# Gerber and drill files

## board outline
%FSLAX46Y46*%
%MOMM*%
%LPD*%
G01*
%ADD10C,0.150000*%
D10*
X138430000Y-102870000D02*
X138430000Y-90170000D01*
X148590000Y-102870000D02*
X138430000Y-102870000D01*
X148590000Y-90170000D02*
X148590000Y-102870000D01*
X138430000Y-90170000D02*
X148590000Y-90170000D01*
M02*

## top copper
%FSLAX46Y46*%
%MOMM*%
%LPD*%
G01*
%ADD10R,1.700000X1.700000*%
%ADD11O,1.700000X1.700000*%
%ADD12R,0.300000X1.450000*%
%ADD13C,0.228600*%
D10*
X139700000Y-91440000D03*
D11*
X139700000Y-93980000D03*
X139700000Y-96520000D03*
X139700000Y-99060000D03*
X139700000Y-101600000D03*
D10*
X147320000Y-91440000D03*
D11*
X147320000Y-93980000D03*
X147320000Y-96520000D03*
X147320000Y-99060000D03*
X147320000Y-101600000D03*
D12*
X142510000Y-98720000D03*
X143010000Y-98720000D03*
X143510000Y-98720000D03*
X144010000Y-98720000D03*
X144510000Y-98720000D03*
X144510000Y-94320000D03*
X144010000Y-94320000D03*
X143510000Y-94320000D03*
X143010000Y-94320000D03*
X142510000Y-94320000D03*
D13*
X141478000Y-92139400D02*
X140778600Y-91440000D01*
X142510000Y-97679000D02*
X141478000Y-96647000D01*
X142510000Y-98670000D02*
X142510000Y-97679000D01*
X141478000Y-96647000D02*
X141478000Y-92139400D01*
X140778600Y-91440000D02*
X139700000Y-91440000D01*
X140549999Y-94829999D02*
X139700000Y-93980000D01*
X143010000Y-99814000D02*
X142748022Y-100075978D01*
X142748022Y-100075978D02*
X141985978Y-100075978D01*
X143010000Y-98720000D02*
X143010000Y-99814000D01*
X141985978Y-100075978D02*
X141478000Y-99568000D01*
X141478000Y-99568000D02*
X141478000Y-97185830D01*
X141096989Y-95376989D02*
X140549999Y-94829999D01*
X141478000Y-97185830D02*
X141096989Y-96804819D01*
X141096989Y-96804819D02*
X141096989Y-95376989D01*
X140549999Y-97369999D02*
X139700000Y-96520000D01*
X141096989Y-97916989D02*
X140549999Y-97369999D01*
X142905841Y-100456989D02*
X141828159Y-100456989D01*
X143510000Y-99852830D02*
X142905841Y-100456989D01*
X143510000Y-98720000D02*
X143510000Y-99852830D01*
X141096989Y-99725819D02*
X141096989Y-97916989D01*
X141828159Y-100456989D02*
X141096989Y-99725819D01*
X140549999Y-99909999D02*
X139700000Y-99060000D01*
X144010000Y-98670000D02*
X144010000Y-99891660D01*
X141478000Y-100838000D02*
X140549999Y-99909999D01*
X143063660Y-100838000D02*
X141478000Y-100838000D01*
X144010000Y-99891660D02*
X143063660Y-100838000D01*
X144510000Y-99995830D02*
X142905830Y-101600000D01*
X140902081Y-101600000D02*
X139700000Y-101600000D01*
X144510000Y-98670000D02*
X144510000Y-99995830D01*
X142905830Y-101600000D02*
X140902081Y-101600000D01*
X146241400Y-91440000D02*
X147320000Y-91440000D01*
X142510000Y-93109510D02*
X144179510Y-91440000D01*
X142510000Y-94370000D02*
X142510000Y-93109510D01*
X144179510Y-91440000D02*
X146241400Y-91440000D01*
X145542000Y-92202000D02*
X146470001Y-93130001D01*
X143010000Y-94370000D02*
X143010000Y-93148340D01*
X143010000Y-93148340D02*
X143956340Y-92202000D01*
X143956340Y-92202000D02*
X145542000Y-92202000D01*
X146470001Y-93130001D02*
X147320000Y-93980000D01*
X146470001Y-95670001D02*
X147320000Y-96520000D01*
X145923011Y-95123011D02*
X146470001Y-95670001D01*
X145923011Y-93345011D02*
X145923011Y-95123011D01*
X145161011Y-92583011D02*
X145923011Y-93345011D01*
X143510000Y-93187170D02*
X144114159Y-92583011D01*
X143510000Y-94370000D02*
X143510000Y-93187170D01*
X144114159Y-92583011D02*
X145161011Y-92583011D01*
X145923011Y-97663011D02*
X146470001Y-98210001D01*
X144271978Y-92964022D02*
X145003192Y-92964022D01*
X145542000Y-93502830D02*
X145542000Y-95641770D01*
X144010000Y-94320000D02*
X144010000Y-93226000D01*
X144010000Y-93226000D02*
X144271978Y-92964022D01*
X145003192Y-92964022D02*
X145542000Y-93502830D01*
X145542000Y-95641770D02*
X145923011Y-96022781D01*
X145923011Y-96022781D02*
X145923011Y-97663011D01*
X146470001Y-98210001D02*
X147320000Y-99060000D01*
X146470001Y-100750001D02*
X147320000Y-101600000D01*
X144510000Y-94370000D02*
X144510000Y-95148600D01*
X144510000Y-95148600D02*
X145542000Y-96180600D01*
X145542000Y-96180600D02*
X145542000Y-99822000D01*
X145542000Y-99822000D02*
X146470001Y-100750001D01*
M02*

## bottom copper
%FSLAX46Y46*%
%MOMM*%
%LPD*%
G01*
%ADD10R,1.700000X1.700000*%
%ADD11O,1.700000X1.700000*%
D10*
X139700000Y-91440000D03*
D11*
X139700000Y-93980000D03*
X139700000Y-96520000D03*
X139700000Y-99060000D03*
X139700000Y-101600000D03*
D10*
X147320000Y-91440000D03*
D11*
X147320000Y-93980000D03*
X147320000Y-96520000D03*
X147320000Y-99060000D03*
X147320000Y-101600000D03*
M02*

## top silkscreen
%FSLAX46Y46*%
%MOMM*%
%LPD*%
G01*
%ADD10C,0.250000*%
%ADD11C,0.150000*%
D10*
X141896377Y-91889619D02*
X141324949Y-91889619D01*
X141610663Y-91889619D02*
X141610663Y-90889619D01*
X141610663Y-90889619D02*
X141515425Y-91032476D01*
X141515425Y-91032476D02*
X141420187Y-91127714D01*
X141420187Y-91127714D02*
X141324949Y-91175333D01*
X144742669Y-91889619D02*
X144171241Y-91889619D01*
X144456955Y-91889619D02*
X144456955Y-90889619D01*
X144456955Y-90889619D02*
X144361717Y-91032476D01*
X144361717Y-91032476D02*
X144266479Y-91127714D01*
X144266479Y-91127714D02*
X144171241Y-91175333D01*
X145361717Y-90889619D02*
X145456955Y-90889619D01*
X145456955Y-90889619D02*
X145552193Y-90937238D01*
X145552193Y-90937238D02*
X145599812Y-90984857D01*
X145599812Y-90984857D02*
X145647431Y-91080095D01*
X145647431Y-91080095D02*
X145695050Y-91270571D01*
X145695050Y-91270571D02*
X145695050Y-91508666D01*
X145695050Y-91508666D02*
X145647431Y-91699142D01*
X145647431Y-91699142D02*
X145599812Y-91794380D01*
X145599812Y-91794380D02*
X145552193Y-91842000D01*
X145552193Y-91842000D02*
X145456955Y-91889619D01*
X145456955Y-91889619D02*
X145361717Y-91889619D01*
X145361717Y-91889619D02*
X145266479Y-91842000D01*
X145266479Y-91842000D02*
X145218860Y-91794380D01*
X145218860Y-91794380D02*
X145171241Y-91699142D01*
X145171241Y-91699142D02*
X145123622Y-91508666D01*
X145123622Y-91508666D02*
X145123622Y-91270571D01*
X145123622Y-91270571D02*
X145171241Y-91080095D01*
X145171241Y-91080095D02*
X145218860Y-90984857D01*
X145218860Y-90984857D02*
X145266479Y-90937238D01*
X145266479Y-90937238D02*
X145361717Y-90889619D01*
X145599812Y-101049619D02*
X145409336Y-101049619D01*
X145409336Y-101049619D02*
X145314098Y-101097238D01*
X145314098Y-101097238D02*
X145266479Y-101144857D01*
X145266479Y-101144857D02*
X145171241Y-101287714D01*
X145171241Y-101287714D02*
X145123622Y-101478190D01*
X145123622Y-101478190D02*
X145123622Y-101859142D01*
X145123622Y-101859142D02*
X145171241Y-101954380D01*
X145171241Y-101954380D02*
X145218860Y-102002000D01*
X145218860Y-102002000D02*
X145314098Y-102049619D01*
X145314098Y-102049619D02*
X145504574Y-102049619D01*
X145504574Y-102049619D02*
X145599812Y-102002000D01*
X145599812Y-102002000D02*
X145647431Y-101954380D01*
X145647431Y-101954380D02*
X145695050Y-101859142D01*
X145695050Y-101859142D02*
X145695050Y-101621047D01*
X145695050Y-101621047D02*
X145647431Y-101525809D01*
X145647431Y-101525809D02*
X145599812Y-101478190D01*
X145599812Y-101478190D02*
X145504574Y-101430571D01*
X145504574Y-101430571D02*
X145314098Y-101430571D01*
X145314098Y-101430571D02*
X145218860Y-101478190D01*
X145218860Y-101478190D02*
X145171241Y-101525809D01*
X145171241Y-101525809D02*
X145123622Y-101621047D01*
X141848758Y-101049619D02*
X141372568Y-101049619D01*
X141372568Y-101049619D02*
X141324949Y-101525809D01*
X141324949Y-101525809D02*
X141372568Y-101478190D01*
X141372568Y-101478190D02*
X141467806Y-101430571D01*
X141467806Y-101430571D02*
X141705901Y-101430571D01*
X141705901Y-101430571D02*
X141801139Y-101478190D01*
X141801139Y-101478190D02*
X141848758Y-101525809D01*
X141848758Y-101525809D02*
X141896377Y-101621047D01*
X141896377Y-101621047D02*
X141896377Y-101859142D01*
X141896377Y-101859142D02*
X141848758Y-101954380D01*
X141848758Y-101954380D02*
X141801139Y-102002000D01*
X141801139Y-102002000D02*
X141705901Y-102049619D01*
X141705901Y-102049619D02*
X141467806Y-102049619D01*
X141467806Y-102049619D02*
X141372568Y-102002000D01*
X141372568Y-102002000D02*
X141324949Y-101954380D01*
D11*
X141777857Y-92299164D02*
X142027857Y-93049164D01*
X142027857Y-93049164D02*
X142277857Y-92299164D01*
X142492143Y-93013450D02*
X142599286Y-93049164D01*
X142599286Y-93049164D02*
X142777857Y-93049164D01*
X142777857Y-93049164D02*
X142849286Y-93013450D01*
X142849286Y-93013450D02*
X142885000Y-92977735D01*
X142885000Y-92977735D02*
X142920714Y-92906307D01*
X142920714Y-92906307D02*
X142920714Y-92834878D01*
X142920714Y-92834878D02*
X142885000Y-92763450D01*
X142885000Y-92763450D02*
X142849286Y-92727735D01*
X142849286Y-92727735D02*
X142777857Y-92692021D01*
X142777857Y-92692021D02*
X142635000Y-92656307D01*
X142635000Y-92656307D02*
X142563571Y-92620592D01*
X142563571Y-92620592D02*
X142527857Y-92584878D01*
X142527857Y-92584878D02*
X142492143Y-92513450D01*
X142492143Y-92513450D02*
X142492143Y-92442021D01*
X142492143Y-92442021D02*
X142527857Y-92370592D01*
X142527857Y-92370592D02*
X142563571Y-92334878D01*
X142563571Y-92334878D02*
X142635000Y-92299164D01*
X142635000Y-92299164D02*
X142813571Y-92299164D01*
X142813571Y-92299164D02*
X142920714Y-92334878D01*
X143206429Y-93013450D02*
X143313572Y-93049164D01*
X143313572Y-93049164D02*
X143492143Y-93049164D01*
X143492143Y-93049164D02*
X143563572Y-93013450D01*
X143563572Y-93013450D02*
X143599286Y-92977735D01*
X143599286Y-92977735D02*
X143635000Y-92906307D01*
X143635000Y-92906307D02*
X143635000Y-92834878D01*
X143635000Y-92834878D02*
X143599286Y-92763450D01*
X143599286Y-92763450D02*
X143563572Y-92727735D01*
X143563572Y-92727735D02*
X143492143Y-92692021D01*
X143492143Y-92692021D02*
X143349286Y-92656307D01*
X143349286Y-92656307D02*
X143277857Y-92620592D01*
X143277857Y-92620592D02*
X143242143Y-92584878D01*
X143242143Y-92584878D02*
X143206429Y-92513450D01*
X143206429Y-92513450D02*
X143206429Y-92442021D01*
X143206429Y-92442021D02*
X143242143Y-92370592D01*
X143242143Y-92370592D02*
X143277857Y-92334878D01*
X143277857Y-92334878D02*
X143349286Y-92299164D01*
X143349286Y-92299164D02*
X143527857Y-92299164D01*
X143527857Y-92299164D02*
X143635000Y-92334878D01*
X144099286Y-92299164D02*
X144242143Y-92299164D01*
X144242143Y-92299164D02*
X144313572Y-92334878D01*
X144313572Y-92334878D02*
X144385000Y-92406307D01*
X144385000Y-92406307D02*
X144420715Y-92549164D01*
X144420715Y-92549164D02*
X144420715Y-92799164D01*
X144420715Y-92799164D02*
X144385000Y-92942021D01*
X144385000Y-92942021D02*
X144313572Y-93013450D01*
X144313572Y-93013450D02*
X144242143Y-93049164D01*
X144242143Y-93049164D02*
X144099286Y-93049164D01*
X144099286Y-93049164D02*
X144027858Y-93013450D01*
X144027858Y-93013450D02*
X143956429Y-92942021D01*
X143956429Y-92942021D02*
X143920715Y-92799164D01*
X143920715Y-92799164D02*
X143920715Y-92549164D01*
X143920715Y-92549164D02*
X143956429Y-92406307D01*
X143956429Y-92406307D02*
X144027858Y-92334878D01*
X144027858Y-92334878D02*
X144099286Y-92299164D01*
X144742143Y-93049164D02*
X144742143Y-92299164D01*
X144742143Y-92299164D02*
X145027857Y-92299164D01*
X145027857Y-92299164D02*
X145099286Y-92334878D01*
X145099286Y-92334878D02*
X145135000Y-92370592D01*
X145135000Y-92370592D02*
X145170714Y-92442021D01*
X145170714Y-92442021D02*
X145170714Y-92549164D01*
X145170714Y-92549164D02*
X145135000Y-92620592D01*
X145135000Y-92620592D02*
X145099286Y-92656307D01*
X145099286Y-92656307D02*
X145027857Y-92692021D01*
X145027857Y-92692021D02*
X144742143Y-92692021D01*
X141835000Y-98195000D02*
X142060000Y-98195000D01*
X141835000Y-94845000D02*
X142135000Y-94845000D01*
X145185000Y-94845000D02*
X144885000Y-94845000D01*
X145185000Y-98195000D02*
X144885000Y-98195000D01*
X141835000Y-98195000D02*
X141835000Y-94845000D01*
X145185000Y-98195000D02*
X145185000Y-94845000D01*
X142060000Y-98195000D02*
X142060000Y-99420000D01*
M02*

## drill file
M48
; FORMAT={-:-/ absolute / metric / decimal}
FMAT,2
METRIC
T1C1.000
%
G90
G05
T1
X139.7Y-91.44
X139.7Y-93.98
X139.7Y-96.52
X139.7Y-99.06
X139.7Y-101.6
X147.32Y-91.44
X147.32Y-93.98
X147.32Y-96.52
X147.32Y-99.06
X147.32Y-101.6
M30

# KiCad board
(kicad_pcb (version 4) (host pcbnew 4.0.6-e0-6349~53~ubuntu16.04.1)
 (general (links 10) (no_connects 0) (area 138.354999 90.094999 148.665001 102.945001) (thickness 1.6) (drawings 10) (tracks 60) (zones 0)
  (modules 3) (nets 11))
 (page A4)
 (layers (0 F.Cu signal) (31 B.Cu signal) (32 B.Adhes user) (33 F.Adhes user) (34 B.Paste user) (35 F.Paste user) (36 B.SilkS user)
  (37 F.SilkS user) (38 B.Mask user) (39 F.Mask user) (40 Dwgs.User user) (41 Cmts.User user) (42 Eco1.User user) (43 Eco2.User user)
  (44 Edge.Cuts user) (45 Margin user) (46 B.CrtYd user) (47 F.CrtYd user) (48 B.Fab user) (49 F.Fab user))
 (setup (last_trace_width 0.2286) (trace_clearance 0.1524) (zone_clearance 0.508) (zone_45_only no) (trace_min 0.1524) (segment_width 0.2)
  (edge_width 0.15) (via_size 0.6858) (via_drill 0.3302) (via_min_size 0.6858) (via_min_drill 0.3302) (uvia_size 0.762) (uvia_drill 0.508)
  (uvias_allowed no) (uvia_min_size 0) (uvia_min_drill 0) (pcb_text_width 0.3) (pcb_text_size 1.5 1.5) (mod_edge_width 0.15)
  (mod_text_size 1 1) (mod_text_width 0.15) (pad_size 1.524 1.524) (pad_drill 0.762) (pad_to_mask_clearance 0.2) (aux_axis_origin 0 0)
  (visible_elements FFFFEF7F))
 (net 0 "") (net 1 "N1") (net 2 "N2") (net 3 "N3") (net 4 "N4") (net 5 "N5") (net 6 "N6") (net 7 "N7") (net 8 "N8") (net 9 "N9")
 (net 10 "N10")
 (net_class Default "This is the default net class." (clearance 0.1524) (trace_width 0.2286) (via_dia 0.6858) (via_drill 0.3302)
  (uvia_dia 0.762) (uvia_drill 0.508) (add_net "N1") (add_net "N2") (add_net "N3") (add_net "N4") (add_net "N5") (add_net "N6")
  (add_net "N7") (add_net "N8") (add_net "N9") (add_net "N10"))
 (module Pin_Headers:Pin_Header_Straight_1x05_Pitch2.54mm (layer B.Cu) (at 139.7 91.44 180)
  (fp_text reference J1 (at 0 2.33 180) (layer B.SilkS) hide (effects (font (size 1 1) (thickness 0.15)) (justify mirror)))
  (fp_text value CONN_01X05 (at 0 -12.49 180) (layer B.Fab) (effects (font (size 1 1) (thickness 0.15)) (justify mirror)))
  (pad 1 thru_hole rect (at 0 0 180) (size 1.7 1.7) (drill 1) (layers *.Cu *.Mask) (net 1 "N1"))
  (pad 2 thru_hole oval (at 0 -2.54 180) (size 1.7 1.7) (drill 1) (layers *.Cu *.Mask) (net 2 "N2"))
  (pad 3 thru_hole oval (at 0 -5.08 180) (size 1.7 1.7) (drill 1) (layers *.Cu *.Mask) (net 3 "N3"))
  (pad 4 thru_hole oval (at 0 -7.62 180) (size 1.7 1.7) (drill 1) (layers *.Cu *.Mask) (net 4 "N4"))
  (pad 5 thru_hole oval (at 0 -10.16 180) (size 1.7 1.7) (drill 1) (layers *.Cu *.Mask) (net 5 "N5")))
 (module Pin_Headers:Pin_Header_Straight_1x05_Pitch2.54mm (layer B.Cu) (at 147.32 91.44 180)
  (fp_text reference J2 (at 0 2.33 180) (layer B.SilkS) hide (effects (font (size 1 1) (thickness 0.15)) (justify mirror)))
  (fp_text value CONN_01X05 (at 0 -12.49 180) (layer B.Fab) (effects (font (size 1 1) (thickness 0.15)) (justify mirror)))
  (pad 1 thru_hole rect (at 0 0 180) (size 1.7 1.7) (drill 1) (layers *.Cu *.Mask) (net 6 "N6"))
  (pad 2 thru_hole oval (at 0 -2.54 180) (size 1.7 1.7) (drill 1) (layers *.Cu *.Mask) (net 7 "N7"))
  (pad 3 thru_hole oval (at 0 -5.08 180) (size 1.7 1.7) (drill 1) (layers *.Cu *.Mask) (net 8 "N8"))
  (pad 4 thru_hole oval (at 0 -7.62 180) (size 1.7 1.7) (drill 1) (layers *.Cu *.Mask) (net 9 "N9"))
  (pad 5 thru_hole oval (at 0 -10.16 180) (size 1.7 1.7) (drill 1) (layers *.Cu *.Mask) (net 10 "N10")))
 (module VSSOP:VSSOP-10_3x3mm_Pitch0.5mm (layer F.Cu) (at 143.51 96.52 90)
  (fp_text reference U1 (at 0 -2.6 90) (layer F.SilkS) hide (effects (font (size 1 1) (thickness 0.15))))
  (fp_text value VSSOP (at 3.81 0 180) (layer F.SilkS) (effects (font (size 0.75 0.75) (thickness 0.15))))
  (fp_line (start -1.675 -1.675) (end -1.675 -1.45) (layer F.SilkS) (width 0.15))
  (fp_line (start 1.675 -1.675) (end 1.675 -1.375) (layer F.SilkS) (width 0.15))
  (fp_line (start 1.675 1.675) (end 1.675 1.375) (layer F.SilkS) (width 0.15))
  (fp_line (start -1.675 1.675) (end -1.675 1.375) (layer F.SilkS) (width 0.15))
  (fp_line (start -1.675 -1.675) (end 1.675 -1.675) (layer F.SilkS) (width 0.15))
  (fp_line (start -1.675 1.675) (end 1.675 1.675) (layer F.SilkS) (width 0.15))
  (fp_line (start -1.675 -1.45) (end -2.9 -1.45) (layer F.SilkS) (width 0.15))
  (pad 1 smd rect (at -2.2 -1 90) (size 1.45 0.3) (layers F.Cu F.Paste F.Mask) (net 1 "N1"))
  (pad 2 smd rect (at -2.2 -0.5 90) (size 1.45 0.3) (layers F.Cu F.Paste F.Mask) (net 2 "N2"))
  (pad 3 smd rect (at -2.2 0 90) (size 1.45 0.3) (layers F.Cu F.Paste F.Mask) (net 3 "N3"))
  (pad 4 smd rect (at -2.2 0.5 90) (size 1.45 0.3) (layers F.Cu F.Paste F.Mask) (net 4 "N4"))
  (pad 5 smd rect (at -2.2 1 90) (size 1.45 0.3) (layers F.Cu F.Paste F.Mask) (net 5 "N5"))
  (pad 6 smd rect (at 2.2 1 90) (size 1.45 0.3) (layers F.Cu F.Paste F.Mask) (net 10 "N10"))
  (pad 7 smd rect (at 2.2 0.5 90) (size 1.45 0.3) (layers F.Cu F.Paste F.Mask) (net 9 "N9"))
  (pad 8 smd rect (at 2.2 0 90) (size 1.45 0.3) (layers F.Cu F.Paste F.Mask) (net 8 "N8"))
  (pad 9 smd rect (at 2.2 -0.5 90) (size 1.45 0.3) (layers F.Cu F.Paste F.Mask) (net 7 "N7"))
  (pad 10 smd rect (at 2.2 -1 90) (size 1.45 0.3) (layers F.Cu F.Paste F.Mask) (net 6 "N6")))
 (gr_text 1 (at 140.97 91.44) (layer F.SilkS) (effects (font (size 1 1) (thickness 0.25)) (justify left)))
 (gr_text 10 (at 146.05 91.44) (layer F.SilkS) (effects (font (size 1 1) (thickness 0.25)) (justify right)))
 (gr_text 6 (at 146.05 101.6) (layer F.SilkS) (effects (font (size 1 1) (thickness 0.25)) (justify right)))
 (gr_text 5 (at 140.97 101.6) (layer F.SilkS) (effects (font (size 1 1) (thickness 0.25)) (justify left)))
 (gr_line (start 138.43 102.87) (end 138.43 90.17) (layer Edge.Cuts) (width 0.15))
 (gr_line (start 148.59 102.87) (end 138.43 102.87) (layer Edge.Cuts) (width 0.15))
 (gr_line (start 148.59 90.17) (end 148.59 102.87) (layer Edge.Cuts) (width 0.15))
 (gr_line (start 138.43 90.17) (end 148.59 90.17) (layer Edge.Cuts) (width 0.15))
 (segment (start 141.478 92.1394) (end 140.7786 91.44) (width 0.2286) (layer F.Cu) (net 1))
 (segment (start 142.51 97.679) (end 141.478 96.647) (width 0.2286) (layer F.Cu) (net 1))
 (segment (start 142.51 98.67) (end 142.51 97.679) (width 0.2286) (layer F.Cu) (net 1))
 (segment (start 141.478 96.647) (end 141.478 92.1394) (width 0.2286) (layer F.Cu) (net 1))
 (segment (start 140.7786 91.44) (end 139.7 91.44) (width 0.2286) (layer F.Cu) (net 1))
 (segment (start 140.549999 94.829999) (end 139.7 93.98) (width 0.2286) (layer F.Cu) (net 2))
 (segment (start 143.01 99.814) (end 142.748022 100.075978) (width 0.2286) (layer F.Cu) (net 2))
 (segment (start 142.748022 100.075978) (end 141.985978 100.075978) (width 0.2286) (layer F.Cu) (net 2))
 (segment (start 143.01 98.72) (end 143.01 99.814) (width 0.2286) (layer F.Cu) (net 2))
 (segment (start 141.985978 100.075978) (end 141.478 99.568) (width 0.2286) (layer F.Cu) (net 2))
 (segment (start 141.478 99.568) (end 141.478 97.18583) (width 0.2286) (layer F.Cu) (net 2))
 (segment (start 141.096989 95.376989) (end 140.549999 94.829999) (width 0.2286) (layer F.Cu) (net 2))
 (segment (start 141.478 97.18583) (end 141.096989 96.804819) (width 0.2286) (layer F.Cu) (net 2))
 (segment (start 141.096989 96.804819) (end 141.096989 95.376989) (width 0.2286) (layer F.Cu) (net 2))
 (segment (start 140.549999 97.369999) (end 139.7 96.52) (width 0.2286) (layer F.Cu) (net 3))
 (segment (start 141.096989 97.916989) (end 140.549999 97.369999) (width 0.2286) (layer F.Cu) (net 3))
 (segment (start 142.905841 100.456989) (end 141.828159 100.456989) (width 0.2286) (layer F.Cu) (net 3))
 (segment (start 143.51 99.85283) (end 142.905841 100.456989) (width 0.2286) (layer F.Cu) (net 3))
 (segment (start 143.51 98.72) (end 143.51 99.85283) (width 0.2286) (layer F.Cu) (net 3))
 (segment (start 141.096989 99.725819) (end 141.096989 97.916989) (width 0.2286) (layer F.Cu) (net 3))
 (segment (start 141.828159 100.456989) (end 141.096989 99.725819) (width 0.2286) (layer F.Cu) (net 3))
 (segment (start 140.549999 99.909999) (end 139.7 99.06) (width 0.2286) (layer F.Cu) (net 4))
 (segment (start 144.01 98.67) (end 144.01 99.89166) (width 0.2286) (layer F.Cu) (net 4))
 (segment (start 141.478 100.838) (end 140.549999 99.909999) (width 0.2286) (layer F.Cu) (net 4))
 (segment (start 143.06366 100.838) (end 141.478 100.838) (width 0.2286) (layer F.Cu) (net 4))
 (segment (start 144.01 99.89166) (end 143.06366 100.838) (width 0.2286) (layer F.Cu) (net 4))
 (segment (start 144.51 99.99583) (end 142.90583 101.6) (width 0.2286) (layer F.Cu) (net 5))
 (segment (start 140.902081 101.6) (end 139.7 101.6) (width 0.2286) (layer F.Cu) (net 5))
 (segment (start 144.51 98.67) (end 144.51 99.99583) (width 0.2286) (layer F.Cu) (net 5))
 (segment (start 142.90583 101.6) (end 140.902081 101.6) (width 0.2286) (layer F.Cu) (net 5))
 (segment (start 146.2414 91.44) (end 147.32 91.44) (width 0.2286) (layer F.Cu) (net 6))
 (segment (start 142.51 93.10951) (end 144.17951 91.44) (width 0.2286) (layer F.Cu) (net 6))
 (segment (start 142.51 94.37) (end 142.51 93.10951) (width 0.2286) (layer F.Cu) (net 6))
 (segment (start 144.17951 91.44) (end 146.2414 91.44) (width 0.2286) (layer F.Cu) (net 6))
 (segment (start 145.542 92.202) (end 146.470001 93.130001) (width 0.2286) (layer F.Cu) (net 7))
 (segment (start 143.01 94.37) (end 143.01 93.14834) (width 0.2286) (layer F.Cu) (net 7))
 (segment (start 143.01 93.14834) (end 143.95634 92.202) (width 0.2286) (layer F.Cu) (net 7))
 (segment (start 143.95634 92.202) (end 145.542 92.202) (width 0.2286) (layer F.Cu) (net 7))
 (segment (start 146.470001 93.130001) (end 147.32 93.98) (width 0.2286) (layer F.Cu) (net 7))
 (segment (start 146.470001 95.670001) (end 147.32 96.52) (width 0.2286) (layer F.Cu) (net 8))
 (segment (start 145.923011 95.123011) (end 146.470001 95.670001) (width 0.2286) (layer F.Cu) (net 8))
 (segment (start 145.923011 93.345011) (end 145.923011 95.123011) (width 0.2286) (layer F.Cu) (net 8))
 (segment (start 145.161011 92.583011) (end 145.923011 93.345011) (width 0.2286) (layer F.Cu) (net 8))
 (segment (start 143.51 93.18717) (end 144.114159 92.583011) (width 0.2286) (layer F.Cu) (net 8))
 (segment (start 143.51 94.37) (end 143.51 93.18717) (width 0.2286) (layer F.Cu) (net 8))
 (segment (start 144.114159 92.583011) (end 145.161011 92.583011) (width 0.2286) (layer F.Cu) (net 8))
 (segment (start 145.923011 97.663011) (end 146.470001 98.210001) (width 0.2286) (layer F.Cu) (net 9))
 (segment (start 144.271978 92.964022) (end 145.003192 92.964022) (width 0.2286) (layer F.Cu) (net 9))
 (segment (start 145.542 93.50283) (end 145.542 95.64177) (width 0.2286) (layer F.Cu) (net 9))
 (segment (start 144.01 94.32) (end 144.01 93.226) (width 0.2286) (layer F.Cu) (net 9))
 (segment (start 144.01 93.226) (end 144.271978 92.964022) (width 0.2286) (layer F.Cu) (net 9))
 (segment (start 145.003192 92.964022) (end 145.542 93.50283) (width 0.2286) (layer F.Cu) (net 9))
 (segment (start 145.542 95.64177) (end 145.923011 96.022781) (width 0.2286) (layer F.Cu) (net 9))
 (segment (start 145.923011 96.022781) (end 145.923011 97.663011) (width 0.2286) (layer F.Cu) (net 9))
 (segment (start 146.470001 98.210001) (end 147.32 99.06) (width 0.2286) (layer F.Cu) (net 9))
 (segment (start 146.470001 100.750001) (end 147.32 101.6) (width 0.2286) (layer F.Cu) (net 10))
 (segment (start 144.51 94.37) (end 144.51 95.1486) (width 0.2286) (layer F.Cu) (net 10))
 (segment (start 144.51 95.1486) (end 145.542 96.1806) (width 0.2286) (layer F.Cu) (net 10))
 (segment (start 145.542 96.1806) (end 145.542 99.822) (width 0.2286) (layer F.Cu) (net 10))
 (segment (start 145.542 99.822) (end 146.470001 100.750001) (width 0.2286) (layer F.Cu) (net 10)))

